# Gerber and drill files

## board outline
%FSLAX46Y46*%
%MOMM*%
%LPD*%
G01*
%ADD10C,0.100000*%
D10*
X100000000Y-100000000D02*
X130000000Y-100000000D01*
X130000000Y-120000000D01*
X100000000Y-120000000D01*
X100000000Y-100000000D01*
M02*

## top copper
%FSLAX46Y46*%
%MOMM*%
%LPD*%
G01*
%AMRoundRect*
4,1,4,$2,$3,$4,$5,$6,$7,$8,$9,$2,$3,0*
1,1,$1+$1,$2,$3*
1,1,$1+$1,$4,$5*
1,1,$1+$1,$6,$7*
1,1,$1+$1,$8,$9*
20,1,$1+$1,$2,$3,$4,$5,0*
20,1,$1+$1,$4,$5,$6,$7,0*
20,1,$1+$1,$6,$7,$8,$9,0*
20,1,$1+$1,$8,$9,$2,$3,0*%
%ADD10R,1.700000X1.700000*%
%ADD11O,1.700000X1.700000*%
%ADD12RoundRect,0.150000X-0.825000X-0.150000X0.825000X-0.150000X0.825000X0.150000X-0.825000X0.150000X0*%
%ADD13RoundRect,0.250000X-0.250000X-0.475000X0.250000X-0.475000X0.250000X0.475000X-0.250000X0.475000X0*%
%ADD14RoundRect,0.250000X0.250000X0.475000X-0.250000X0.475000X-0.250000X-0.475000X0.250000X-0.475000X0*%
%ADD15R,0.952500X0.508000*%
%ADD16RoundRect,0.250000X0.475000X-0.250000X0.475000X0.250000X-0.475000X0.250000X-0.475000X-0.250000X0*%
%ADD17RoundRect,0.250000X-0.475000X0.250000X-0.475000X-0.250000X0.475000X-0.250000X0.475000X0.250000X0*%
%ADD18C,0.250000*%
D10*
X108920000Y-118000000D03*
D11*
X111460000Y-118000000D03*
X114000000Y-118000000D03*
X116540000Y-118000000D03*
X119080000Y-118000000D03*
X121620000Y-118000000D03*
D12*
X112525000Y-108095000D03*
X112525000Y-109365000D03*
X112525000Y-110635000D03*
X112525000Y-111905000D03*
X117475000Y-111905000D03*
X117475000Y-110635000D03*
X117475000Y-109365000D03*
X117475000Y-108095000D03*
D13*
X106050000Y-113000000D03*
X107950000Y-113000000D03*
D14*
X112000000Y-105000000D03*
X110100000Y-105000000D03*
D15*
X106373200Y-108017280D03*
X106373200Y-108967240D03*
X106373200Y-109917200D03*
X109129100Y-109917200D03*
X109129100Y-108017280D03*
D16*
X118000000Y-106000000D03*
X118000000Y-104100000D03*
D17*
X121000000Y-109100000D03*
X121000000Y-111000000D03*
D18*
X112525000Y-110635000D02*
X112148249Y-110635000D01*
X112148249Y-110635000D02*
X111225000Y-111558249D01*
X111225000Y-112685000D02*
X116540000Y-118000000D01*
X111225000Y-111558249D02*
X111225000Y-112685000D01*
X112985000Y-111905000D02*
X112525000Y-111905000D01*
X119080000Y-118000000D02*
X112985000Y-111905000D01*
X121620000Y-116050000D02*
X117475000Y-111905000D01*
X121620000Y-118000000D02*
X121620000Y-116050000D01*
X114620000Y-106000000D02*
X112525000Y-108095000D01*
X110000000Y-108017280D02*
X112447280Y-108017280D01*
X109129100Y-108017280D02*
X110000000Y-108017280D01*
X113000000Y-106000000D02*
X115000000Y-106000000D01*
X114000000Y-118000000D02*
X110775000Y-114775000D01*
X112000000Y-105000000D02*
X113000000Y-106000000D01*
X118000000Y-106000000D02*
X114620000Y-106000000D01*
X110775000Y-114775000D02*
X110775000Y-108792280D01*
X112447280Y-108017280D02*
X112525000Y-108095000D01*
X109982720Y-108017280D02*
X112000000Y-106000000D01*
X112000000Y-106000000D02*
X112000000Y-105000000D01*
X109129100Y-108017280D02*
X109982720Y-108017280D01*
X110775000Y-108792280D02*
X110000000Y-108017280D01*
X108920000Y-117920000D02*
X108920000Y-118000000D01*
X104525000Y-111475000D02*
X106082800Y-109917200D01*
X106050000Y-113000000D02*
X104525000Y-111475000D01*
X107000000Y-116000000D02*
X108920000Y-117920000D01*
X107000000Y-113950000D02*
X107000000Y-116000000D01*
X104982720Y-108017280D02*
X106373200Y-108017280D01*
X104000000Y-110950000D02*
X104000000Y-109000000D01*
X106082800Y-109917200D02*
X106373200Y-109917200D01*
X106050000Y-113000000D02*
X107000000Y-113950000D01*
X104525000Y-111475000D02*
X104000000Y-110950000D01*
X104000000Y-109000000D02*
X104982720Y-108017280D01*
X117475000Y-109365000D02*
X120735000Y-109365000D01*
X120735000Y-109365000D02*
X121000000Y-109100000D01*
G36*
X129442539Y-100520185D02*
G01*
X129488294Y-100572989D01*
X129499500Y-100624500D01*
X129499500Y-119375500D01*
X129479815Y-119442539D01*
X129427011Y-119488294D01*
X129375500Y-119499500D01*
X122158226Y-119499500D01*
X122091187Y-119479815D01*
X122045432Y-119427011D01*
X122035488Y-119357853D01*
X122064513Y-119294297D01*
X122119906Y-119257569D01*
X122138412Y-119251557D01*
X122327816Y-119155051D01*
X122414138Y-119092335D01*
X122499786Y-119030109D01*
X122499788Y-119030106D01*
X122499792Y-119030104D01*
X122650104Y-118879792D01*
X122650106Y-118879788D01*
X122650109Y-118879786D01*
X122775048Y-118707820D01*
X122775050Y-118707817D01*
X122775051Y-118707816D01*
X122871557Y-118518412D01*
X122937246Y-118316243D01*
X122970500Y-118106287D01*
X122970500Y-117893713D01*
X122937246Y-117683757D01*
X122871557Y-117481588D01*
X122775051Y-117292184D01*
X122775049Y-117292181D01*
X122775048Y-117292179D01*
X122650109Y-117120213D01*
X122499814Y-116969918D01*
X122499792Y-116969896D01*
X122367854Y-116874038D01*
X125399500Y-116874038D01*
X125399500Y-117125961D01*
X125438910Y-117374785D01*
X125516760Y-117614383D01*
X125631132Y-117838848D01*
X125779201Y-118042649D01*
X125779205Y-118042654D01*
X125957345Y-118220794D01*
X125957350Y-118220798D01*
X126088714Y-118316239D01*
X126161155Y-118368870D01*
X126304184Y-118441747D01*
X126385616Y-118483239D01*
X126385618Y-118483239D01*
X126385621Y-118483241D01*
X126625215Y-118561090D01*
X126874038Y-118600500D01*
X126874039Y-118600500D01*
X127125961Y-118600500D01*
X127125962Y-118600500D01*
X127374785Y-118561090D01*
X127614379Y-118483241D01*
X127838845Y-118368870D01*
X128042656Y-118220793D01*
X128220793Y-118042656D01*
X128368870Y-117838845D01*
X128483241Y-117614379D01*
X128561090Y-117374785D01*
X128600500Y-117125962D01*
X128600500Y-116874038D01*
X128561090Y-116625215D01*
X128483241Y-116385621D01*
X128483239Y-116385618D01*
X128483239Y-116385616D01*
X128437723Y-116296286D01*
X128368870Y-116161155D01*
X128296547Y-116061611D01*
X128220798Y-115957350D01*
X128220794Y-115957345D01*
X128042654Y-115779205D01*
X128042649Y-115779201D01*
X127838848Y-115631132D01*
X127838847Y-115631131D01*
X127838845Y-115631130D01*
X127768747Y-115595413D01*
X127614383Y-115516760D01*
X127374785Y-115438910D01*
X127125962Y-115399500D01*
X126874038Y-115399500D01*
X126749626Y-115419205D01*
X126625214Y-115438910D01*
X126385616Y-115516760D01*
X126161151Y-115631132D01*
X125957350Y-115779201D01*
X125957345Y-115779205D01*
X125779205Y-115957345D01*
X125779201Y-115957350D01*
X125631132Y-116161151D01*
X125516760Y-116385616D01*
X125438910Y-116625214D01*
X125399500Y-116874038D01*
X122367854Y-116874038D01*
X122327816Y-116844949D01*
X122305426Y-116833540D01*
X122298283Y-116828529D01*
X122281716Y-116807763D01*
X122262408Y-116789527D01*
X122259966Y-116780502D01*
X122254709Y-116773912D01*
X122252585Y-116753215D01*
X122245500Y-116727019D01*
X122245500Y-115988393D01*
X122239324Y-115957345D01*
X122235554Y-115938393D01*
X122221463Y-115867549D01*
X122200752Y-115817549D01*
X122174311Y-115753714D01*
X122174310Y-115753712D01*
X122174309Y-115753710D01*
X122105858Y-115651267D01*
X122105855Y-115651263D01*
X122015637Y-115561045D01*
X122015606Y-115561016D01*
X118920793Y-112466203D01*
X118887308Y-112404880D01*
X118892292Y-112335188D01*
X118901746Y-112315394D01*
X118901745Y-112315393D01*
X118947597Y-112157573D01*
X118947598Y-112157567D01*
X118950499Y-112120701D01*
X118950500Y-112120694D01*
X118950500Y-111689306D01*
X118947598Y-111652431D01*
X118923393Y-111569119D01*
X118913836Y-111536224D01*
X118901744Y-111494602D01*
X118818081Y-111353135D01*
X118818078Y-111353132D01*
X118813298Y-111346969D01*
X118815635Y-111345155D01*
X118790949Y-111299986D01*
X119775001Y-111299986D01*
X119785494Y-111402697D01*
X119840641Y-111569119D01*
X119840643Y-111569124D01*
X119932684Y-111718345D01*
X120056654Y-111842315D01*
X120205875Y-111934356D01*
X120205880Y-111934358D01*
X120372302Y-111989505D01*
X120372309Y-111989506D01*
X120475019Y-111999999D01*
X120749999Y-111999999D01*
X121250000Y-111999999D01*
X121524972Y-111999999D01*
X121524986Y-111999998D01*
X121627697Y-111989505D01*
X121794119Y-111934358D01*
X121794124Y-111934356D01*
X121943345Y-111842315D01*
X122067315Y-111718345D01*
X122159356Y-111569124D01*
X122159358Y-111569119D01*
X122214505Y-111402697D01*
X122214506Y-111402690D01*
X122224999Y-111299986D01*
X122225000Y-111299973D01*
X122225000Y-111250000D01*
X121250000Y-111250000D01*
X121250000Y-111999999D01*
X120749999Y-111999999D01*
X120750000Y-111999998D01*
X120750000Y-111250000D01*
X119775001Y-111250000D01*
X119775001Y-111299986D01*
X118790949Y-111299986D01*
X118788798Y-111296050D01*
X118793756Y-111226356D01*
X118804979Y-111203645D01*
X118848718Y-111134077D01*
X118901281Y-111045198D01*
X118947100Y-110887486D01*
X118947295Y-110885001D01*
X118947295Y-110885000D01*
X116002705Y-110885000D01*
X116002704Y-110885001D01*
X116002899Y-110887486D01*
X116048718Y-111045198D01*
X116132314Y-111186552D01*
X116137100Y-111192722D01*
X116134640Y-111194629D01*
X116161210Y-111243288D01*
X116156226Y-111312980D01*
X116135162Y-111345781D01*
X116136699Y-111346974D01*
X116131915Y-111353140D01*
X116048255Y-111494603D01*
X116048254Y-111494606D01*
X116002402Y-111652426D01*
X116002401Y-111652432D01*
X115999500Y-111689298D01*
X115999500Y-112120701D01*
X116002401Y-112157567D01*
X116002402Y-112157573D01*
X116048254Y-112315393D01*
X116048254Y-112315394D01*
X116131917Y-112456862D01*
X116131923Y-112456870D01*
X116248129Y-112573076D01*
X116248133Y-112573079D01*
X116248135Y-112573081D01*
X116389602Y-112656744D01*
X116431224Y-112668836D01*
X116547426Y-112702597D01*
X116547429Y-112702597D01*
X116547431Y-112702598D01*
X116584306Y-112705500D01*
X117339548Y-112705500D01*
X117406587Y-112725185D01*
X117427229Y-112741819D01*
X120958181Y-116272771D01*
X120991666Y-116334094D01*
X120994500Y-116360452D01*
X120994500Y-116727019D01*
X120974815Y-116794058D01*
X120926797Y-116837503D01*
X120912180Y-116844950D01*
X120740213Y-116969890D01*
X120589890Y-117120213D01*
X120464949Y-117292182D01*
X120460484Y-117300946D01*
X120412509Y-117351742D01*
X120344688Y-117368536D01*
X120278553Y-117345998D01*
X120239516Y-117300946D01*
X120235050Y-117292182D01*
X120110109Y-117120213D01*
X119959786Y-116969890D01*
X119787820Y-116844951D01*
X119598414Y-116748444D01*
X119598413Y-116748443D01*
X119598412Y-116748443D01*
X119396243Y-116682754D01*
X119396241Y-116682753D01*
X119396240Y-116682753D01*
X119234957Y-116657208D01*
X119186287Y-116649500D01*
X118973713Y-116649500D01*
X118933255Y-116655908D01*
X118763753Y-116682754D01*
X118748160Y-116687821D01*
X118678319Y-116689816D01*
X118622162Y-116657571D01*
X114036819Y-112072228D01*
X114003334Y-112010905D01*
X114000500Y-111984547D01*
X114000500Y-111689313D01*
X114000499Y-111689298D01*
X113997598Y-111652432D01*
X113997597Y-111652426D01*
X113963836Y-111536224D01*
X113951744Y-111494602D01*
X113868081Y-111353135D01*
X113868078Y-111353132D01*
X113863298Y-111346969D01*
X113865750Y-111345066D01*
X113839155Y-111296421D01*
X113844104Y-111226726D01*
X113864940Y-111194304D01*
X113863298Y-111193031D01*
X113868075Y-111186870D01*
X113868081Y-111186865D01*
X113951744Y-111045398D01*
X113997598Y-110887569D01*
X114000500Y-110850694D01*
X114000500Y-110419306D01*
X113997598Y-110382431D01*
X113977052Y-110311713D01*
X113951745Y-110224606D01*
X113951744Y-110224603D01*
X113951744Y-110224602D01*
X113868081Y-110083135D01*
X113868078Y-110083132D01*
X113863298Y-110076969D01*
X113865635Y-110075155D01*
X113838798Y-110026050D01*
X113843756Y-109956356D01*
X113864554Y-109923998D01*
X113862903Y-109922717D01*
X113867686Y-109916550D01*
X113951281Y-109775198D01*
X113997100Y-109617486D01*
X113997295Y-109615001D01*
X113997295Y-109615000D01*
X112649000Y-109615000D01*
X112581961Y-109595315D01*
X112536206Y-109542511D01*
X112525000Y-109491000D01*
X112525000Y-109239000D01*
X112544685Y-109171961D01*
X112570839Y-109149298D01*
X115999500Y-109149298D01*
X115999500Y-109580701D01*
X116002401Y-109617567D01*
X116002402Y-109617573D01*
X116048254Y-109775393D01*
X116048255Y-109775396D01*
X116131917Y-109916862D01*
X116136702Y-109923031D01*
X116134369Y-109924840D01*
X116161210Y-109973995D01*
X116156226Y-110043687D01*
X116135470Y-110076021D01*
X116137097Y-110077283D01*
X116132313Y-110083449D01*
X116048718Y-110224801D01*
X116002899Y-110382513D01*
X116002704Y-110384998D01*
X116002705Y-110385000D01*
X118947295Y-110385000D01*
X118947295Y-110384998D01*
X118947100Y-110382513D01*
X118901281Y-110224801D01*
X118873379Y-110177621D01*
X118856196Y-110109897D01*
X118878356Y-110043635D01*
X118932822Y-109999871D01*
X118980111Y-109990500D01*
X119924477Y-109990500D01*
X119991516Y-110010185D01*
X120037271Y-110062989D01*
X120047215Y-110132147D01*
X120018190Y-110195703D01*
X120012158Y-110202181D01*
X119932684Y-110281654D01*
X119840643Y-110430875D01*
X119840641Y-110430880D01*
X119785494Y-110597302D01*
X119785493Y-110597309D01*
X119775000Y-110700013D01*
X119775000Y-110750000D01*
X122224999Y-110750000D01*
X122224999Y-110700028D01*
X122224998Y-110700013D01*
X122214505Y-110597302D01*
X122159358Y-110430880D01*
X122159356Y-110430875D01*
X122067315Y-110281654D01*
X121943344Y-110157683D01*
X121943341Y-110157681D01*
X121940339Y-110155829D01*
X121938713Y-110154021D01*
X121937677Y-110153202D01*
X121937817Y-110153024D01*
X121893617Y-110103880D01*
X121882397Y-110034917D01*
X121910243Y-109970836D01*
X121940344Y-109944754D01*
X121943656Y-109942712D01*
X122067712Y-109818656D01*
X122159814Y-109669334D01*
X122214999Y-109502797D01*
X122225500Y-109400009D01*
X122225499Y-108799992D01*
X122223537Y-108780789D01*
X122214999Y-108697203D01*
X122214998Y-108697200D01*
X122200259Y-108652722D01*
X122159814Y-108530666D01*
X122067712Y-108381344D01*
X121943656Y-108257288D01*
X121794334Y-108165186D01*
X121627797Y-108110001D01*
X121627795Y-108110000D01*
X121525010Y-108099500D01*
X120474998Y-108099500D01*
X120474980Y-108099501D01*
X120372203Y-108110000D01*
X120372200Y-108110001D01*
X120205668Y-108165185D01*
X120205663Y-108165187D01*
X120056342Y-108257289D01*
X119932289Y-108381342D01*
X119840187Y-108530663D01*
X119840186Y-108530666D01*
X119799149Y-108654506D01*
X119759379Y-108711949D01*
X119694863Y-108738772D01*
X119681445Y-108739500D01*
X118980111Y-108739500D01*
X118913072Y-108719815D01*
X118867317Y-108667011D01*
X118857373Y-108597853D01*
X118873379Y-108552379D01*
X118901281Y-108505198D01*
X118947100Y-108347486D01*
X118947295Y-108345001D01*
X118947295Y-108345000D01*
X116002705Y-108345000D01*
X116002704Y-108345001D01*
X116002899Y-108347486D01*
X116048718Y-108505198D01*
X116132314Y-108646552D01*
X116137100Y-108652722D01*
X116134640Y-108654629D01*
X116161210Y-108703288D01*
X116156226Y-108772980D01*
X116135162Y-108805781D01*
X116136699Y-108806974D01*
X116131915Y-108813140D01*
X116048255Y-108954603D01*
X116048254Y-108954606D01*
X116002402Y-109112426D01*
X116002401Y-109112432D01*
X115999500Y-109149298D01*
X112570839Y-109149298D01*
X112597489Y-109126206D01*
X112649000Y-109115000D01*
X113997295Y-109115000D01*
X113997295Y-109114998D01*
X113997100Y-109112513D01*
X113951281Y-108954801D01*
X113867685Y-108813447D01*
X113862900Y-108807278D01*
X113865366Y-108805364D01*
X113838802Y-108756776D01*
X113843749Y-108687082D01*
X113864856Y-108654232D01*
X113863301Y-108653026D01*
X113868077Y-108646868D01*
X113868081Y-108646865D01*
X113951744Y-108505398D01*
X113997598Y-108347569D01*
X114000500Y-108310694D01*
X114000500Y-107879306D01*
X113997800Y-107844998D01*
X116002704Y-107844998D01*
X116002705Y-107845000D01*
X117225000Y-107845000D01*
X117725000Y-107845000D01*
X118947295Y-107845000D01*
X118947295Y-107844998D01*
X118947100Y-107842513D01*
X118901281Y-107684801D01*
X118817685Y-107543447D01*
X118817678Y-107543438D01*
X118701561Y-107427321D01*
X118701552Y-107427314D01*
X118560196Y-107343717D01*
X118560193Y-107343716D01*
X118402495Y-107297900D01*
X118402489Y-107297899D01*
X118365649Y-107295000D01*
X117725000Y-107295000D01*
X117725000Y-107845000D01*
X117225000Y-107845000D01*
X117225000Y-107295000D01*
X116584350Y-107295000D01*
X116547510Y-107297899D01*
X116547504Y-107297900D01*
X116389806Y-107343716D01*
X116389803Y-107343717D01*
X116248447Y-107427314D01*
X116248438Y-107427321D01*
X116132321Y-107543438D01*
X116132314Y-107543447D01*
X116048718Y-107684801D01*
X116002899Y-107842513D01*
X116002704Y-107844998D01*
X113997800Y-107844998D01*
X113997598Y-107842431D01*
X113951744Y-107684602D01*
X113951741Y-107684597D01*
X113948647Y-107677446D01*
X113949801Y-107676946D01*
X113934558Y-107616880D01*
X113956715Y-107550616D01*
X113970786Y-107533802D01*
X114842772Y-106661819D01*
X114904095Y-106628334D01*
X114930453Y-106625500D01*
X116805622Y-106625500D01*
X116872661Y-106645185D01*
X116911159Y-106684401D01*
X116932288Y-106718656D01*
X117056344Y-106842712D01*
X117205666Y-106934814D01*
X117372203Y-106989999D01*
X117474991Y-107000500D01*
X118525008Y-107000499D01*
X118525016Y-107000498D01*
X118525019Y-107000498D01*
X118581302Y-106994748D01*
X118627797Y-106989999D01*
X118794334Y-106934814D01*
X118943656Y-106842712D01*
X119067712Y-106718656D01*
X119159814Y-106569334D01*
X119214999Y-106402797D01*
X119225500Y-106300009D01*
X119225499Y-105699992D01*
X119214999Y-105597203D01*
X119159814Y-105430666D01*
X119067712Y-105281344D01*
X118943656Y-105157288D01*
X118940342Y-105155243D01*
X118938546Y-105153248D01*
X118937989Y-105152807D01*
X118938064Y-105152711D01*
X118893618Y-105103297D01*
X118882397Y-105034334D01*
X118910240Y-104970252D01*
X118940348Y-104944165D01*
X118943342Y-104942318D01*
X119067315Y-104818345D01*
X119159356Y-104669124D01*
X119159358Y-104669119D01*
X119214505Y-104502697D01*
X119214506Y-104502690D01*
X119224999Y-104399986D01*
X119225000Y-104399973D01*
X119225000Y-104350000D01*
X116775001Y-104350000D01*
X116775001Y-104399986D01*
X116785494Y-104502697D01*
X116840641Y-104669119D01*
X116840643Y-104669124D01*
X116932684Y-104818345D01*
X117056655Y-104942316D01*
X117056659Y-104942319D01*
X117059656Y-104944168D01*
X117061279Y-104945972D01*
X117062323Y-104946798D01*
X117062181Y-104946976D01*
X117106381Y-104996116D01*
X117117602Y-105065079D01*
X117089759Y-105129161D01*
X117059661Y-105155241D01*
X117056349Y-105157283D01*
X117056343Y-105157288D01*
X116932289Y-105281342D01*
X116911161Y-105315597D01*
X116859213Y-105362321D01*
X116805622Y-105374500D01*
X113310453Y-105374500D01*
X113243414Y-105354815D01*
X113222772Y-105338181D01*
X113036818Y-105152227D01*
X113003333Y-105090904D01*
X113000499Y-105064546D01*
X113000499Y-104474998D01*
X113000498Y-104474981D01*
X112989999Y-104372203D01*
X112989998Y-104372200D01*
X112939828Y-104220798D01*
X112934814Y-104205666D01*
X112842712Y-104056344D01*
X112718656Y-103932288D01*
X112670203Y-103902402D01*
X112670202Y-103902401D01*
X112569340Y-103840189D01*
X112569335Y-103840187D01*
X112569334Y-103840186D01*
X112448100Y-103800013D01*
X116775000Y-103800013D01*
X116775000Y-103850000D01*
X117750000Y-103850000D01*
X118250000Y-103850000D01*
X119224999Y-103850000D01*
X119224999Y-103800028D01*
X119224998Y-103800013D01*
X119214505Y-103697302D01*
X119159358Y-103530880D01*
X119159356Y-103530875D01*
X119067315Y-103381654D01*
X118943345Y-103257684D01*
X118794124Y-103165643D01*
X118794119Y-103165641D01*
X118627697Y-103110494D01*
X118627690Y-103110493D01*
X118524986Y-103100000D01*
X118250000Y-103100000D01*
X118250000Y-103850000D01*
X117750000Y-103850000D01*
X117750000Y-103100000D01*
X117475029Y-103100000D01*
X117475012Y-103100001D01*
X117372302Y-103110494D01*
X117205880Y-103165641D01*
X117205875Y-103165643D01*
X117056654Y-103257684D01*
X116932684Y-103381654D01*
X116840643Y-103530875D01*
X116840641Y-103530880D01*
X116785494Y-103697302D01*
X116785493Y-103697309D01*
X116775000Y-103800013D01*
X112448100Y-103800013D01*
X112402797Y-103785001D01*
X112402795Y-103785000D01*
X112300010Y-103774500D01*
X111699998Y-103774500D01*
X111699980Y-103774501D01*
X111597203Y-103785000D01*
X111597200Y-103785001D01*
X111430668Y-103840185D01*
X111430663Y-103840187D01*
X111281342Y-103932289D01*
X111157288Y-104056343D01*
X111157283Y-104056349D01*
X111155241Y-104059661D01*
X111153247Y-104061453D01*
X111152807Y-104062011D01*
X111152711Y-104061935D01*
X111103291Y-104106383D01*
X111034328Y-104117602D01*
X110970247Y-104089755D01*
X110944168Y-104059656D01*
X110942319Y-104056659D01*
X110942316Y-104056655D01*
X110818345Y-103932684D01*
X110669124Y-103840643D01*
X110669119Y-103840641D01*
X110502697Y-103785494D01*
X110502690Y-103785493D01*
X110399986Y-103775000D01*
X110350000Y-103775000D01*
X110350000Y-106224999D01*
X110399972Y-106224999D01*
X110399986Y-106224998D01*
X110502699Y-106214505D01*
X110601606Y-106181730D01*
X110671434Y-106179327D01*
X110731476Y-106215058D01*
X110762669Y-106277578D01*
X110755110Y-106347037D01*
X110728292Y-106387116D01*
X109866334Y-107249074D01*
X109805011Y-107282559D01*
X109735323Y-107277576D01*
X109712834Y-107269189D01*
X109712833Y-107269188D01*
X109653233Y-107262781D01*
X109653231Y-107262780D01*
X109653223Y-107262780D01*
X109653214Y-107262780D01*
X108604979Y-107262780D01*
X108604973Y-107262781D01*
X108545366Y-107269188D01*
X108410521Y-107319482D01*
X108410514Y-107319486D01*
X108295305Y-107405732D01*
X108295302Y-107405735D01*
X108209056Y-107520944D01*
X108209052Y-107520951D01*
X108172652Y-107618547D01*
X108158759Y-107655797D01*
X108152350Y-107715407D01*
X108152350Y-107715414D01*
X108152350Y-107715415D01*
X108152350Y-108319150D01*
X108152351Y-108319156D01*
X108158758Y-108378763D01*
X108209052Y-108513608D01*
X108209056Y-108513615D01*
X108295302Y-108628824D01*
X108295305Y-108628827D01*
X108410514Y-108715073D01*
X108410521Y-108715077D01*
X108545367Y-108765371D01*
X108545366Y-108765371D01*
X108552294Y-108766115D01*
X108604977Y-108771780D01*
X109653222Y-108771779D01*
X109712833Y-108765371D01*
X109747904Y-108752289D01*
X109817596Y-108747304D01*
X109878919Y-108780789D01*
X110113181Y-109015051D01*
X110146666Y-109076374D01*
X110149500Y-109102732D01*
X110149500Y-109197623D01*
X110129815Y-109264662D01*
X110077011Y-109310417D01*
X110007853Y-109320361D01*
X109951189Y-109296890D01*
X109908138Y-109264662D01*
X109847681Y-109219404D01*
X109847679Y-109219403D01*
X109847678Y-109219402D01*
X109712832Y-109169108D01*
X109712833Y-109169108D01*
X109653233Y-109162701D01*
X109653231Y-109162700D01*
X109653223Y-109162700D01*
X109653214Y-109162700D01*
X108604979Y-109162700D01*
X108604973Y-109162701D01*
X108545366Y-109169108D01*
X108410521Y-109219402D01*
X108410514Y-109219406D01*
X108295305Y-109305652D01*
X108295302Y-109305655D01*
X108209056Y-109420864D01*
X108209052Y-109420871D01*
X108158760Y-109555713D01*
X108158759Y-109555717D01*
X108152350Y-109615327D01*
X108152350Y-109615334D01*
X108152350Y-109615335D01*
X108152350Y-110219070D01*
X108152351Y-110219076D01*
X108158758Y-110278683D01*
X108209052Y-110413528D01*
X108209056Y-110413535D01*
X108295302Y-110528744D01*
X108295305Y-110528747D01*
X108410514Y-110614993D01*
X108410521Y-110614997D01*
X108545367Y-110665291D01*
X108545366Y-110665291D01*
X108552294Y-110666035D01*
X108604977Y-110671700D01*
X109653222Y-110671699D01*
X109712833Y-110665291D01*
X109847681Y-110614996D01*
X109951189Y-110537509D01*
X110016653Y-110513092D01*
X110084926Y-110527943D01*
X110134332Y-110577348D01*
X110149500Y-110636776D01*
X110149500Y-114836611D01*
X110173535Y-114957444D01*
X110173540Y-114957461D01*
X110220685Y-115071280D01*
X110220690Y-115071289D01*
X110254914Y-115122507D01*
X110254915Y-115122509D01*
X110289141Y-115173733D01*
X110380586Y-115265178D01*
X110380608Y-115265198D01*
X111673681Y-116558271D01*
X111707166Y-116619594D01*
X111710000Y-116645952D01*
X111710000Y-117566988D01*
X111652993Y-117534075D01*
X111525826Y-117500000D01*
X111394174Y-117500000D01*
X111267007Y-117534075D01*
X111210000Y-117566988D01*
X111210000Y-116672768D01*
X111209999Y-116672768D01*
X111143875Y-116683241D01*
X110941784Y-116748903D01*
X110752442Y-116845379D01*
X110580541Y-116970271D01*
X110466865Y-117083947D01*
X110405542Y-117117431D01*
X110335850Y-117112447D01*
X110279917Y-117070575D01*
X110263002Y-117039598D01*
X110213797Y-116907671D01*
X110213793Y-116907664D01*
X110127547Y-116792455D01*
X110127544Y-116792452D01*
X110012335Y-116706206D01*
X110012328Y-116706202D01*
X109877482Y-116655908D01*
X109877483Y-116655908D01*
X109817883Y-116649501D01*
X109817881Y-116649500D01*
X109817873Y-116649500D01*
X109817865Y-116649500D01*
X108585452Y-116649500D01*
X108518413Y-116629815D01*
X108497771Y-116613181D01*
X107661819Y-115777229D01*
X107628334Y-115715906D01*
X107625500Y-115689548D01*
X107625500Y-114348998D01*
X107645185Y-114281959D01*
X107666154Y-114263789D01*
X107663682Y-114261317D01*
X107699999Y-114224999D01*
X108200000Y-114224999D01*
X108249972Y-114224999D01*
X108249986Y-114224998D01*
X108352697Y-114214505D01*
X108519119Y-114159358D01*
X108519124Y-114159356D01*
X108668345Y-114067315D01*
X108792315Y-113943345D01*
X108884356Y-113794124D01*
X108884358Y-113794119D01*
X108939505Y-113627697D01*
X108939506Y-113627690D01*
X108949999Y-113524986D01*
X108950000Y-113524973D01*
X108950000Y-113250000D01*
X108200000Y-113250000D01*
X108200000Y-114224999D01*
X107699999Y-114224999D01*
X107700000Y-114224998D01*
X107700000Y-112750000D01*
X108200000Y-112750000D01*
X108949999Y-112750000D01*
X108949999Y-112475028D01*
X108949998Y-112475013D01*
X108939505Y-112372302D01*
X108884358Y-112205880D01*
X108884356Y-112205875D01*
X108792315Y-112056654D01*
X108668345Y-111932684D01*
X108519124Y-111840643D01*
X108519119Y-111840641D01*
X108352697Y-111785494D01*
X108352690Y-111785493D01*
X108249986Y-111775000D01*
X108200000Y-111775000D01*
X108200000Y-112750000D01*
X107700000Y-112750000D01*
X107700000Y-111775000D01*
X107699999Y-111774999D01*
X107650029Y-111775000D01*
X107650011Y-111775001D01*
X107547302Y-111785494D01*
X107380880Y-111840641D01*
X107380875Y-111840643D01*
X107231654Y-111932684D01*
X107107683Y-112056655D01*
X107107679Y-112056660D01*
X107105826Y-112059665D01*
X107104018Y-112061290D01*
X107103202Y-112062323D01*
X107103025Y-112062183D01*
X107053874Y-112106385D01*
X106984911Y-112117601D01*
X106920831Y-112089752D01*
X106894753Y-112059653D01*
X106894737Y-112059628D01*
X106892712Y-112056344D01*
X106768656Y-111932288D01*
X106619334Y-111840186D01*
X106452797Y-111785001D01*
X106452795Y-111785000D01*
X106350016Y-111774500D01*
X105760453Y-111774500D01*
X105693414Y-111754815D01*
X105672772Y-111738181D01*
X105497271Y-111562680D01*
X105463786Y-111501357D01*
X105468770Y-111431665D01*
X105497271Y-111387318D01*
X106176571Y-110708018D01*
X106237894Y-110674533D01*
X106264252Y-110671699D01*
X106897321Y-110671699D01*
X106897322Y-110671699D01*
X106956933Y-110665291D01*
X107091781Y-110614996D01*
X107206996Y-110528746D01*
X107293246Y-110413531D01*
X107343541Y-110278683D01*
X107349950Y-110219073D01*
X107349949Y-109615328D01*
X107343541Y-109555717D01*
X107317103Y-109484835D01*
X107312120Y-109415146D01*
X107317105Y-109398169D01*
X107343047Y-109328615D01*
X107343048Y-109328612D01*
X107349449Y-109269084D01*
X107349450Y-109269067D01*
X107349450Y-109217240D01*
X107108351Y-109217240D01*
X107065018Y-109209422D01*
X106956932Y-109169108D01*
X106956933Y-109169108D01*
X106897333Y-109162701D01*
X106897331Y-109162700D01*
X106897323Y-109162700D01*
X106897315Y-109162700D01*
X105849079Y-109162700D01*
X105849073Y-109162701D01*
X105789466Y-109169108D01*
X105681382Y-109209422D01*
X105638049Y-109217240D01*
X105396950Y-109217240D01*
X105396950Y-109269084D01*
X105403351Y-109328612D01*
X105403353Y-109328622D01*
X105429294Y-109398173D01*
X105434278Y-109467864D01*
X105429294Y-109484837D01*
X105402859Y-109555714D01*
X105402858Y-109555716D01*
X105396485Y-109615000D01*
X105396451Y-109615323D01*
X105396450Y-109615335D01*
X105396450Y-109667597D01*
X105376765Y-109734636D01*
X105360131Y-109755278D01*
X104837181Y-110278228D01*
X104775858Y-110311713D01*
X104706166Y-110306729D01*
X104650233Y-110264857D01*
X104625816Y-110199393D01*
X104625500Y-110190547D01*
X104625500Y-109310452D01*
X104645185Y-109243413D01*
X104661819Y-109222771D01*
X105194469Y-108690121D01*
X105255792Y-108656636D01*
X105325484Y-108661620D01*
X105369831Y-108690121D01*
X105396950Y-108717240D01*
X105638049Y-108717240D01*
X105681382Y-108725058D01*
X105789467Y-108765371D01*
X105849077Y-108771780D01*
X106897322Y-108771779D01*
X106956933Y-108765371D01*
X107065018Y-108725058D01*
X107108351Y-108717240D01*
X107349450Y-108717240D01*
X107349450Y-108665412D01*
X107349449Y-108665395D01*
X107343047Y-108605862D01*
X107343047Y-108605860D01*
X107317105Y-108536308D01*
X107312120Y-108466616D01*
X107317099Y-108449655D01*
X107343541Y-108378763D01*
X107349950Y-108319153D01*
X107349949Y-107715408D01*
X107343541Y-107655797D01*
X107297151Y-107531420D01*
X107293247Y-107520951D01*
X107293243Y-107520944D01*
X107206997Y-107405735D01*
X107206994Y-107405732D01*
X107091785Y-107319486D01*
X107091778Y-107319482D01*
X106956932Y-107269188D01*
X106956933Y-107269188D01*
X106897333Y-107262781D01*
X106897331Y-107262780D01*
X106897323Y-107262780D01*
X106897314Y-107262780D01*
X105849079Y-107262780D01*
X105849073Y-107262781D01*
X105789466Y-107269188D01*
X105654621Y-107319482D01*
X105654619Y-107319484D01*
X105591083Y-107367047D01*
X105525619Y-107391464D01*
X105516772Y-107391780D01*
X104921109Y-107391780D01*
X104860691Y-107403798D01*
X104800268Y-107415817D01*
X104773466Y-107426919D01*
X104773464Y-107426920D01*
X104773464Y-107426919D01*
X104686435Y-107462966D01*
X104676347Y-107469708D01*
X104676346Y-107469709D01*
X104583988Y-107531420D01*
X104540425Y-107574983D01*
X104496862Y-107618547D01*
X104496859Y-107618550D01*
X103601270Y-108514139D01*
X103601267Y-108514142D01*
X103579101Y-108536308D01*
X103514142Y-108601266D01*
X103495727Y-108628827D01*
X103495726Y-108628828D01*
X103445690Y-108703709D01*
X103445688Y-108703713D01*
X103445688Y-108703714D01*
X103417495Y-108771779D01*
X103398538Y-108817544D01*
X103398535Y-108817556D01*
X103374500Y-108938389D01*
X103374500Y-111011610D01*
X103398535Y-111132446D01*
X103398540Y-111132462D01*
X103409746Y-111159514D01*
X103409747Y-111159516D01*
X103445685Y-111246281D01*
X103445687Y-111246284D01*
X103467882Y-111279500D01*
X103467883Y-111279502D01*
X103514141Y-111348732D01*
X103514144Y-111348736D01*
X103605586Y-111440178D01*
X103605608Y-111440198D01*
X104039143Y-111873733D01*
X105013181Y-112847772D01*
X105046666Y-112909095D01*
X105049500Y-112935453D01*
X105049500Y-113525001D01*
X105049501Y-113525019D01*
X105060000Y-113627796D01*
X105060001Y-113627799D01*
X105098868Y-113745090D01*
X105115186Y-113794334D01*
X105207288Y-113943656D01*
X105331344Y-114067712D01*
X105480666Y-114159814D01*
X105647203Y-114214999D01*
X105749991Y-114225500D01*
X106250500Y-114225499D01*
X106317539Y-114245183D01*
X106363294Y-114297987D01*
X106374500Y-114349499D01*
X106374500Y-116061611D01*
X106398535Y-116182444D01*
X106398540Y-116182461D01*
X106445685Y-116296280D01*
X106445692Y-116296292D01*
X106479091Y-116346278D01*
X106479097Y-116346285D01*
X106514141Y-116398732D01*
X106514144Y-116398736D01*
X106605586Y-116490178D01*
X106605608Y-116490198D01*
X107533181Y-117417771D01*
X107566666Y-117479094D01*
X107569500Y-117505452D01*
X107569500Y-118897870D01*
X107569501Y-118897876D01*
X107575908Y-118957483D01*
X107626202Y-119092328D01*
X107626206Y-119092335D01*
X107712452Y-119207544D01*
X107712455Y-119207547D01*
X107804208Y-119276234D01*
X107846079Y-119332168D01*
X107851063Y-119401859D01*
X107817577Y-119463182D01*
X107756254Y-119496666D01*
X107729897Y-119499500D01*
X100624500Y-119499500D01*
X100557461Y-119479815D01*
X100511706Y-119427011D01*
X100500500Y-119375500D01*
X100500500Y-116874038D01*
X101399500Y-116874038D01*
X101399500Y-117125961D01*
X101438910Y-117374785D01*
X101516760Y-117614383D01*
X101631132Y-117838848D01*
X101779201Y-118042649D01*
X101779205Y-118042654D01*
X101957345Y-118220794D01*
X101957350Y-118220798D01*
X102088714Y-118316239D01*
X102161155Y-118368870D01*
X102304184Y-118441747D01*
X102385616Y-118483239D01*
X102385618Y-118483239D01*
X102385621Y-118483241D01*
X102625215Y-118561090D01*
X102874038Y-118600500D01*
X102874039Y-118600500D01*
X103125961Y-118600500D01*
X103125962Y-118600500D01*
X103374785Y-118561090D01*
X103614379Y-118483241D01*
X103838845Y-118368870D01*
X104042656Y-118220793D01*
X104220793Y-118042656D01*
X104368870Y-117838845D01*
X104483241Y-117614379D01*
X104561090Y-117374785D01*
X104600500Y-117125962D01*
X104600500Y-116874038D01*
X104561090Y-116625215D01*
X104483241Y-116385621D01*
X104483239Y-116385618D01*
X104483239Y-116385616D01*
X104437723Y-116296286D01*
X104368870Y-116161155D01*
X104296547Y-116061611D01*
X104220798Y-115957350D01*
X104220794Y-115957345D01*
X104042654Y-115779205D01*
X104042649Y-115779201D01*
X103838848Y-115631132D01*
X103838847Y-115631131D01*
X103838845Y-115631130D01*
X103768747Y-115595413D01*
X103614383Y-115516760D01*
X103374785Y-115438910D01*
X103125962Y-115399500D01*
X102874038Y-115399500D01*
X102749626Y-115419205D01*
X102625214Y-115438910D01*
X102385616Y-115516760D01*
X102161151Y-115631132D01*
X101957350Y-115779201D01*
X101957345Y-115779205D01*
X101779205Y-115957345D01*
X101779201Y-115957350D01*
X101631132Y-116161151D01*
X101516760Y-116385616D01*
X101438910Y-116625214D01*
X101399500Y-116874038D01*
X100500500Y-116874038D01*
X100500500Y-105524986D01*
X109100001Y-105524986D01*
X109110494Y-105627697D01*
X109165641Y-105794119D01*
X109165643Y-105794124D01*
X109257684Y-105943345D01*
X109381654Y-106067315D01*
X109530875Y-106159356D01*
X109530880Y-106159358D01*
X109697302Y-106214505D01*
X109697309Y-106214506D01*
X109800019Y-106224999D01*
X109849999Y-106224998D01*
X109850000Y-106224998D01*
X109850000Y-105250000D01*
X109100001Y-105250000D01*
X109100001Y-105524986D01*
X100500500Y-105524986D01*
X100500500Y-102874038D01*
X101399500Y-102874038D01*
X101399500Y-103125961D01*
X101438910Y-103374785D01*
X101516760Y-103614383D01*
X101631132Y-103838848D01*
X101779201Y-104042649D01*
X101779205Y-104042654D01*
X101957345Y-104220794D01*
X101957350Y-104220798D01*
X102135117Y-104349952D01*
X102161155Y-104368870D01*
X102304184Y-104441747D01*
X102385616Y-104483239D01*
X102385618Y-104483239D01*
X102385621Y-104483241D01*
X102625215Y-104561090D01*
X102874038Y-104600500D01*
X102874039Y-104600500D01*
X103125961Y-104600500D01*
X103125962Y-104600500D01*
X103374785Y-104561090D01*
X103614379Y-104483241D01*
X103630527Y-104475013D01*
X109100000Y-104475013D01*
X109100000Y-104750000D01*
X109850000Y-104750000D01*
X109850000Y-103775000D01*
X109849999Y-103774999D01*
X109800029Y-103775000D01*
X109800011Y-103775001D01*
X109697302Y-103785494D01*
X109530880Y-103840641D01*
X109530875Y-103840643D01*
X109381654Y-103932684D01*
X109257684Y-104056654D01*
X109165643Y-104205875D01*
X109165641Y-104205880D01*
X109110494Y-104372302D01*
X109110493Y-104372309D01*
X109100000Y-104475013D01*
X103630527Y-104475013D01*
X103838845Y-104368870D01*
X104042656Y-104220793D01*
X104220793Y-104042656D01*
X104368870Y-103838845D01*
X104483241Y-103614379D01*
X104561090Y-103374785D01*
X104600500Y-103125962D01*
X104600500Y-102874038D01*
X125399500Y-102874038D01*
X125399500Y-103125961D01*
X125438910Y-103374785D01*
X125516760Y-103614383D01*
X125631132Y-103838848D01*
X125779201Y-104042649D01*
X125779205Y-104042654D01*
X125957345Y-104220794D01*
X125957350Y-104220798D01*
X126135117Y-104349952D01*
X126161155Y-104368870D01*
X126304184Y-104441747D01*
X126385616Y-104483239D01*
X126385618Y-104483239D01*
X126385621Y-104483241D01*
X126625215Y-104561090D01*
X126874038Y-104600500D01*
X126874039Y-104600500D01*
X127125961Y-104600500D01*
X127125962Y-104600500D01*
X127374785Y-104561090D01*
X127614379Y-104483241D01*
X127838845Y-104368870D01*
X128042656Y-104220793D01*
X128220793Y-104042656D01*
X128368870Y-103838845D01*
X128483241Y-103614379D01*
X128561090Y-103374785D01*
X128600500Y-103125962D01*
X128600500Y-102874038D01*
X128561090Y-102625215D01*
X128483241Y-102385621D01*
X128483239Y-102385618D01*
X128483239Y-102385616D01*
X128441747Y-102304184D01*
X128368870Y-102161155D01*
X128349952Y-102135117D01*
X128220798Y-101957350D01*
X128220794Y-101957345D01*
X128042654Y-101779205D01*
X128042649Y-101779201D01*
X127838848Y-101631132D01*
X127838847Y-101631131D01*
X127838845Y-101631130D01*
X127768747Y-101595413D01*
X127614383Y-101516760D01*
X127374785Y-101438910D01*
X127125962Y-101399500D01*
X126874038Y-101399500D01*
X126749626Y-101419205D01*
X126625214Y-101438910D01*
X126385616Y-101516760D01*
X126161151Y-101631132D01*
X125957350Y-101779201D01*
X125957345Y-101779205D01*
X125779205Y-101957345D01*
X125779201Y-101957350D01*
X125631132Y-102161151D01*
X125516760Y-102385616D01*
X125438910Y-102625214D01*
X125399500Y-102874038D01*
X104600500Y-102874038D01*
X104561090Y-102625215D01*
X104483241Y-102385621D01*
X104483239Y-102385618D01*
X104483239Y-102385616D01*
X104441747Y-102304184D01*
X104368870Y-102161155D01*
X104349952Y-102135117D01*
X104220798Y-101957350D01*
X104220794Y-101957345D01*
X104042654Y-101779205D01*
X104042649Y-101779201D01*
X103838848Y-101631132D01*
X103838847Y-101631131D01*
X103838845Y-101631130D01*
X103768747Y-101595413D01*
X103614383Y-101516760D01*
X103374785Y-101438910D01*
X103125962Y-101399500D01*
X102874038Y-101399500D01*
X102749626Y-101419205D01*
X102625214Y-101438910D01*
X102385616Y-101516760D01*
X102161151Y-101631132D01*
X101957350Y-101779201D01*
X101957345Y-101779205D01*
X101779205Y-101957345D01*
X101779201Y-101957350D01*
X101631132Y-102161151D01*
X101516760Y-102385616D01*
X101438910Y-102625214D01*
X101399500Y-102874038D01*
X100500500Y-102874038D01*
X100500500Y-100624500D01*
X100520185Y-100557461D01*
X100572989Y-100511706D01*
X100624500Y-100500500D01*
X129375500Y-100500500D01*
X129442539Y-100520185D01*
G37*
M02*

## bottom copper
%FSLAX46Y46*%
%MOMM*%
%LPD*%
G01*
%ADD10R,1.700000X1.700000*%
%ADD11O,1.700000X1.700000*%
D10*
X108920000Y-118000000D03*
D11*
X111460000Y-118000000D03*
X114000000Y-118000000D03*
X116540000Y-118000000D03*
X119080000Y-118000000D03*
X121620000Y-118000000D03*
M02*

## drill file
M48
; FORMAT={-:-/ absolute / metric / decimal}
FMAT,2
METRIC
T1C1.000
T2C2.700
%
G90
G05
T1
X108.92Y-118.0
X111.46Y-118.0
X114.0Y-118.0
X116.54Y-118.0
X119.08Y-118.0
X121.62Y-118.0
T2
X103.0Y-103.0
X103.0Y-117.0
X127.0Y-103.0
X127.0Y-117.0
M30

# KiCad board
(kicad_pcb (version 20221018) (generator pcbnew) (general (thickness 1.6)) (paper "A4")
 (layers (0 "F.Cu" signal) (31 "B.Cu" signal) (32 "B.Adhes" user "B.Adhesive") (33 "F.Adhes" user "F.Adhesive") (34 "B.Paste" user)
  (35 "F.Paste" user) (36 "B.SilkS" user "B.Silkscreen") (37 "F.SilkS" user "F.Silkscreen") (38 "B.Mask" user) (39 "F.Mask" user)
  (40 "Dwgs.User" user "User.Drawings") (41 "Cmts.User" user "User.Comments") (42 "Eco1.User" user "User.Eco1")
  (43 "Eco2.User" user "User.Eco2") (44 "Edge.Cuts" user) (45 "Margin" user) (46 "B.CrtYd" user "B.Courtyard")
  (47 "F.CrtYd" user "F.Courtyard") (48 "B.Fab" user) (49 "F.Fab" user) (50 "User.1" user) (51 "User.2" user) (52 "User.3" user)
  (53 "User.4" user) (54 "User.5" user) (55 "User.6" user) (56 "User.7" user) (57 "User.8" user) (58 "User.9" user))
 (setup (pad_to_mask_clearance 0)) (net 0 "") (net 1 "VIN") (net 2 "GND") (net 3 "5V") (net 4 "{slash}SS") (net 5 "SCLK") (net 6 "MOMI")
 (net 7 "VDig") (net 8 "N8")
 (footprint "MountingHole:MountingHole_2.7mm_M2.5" (layer "F.Cu") (at 103 117)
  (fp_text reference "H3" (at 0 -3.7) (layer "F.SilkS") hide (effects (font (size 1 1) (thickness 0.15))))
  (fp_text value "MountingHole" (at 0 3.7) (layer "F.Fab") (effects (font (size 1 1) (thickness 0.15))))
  (pad "" np_thru_hole circle (at 0 0) (size 2.7 2.7) (drill 2.7) (layers "*.Cu" "*.Mask")))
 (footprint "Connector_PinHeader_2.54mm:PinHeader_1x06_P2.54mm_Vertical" (layer "F.Cu") (at 108.92 118 90)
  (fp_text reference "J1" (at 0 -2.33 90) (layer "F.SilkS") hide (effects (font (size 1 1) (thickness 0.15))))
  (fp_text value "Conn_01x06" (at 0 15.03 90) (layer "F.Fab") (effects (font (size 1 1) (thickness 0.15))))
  (pad "1" thru_hole rect (at 0 0 90) (size 1.7 1.7) (drill 1) (layers "*.Cu" "*.Mask") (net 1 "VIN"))
  (pad "2" thru_hole oval (at 0 2.54 90) (size 1.7 1.7) (drill 1) (layers "*.Cu" "*.Mask") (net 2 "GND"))
  (pad "3" thru_hole oval (at 0 5.08 90) (size 1.7 1.7) (drill 1) (layers "*.Cu" "*.Mask") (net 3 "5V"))
  (pad "4" thru_hole oval (at 0 7.62 90) (size 1.7 1.7) (drill 1) (layers "*.Cu" "*.Mask") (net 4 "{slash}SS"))
  (pad "5" thru_hole oval (at 0 10.16 90) (size 1.7 1.7) (drill 1) (layers "*.Cu" "*.Mask") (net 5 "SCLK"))
  (pad "6" thru_hole oval (at 0 12.7 90) (size 1.7 1.7) (drill 1) (layers "*.Cu" "*.Mask") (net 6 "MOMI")))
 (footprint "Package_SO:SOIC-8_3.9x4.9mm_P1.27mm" (layer "F.Cu") (at 115 110)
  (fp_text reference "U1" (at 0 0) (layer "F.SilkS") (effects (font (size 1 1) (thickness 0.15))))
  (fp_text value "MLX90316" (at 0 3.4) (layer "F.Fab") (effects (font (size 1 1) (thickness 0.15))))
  (pad "1" smd roundrect (at -2.475 -1.905) (size 1.95 0.6) (layers "F.Cu" "F.Paste" "F.Mask") (roundrect_rratio 0.25) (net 3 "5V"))
  (pad "2" smd roundrect (at -2.475 -0.635) (size 1.95 0.6) (layers "F.Cu" "F.Paste" "F.Mask") (roundrect_rratio 0.25) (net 2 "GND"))
  (pad "3" smd roundrect (at -2.475 0.635) (size 1.95 0.6) (layers "F.Cu" "F.Paste" "F.Mask") (roundrect_rratio 0.25) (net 4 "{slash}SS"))
  (pad "4" smd roundrect (at -2.475 1.905) (size 1.95 0.6) (layers "F.Cu" "F.Paste" "F.Mask") (roundrect_rratio 0.25) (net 5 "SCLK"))
  (pad "5" smd roundrect (at 2.475 1.905) (size 1.95 0.6) (layers "F.Cu" "F.Paste" "F.Mask") (roundrect_rratio 0.25) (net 6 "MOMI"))
  (pad "6" smd roundrect (at 2.475 0.635) (size 1.95 0.6) (layers "F.Cu" "F.Paste" "F.Mask") (roundrect_rratio 0.25) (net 2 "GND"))
  (pad "7" smd roundrect (at 2.475 -0.635) (size 1.95 0.6) (layers "F.Cu" "F.Paste" "F.Mask") (roundrect_rratio 0.25) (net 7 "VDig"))
  (pad "8" smd roundrect (at 2.475 -1.905) (size 1.95 0.6) (layers "F.Cu" "F.Paste" "F.Mask") (roundrect_rratio 0.25) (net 2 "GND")))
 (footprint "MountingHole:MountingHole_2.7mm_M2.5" (layer "F.Cu") (at 127 103)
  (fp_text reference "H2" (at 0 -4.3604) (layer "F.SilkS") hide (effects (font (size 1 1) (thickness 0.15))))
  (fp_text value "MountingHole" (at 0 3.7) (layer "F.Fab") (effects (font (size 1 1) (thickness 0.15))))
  (pad "" np_thru_hole circle (at 0 0) (size 2.7 2.7) (drill 2.7) (layers "*.Cu" "*.Mask")))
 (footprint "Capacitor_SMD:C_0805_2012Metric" (layer "F.Cu") (at 107 113)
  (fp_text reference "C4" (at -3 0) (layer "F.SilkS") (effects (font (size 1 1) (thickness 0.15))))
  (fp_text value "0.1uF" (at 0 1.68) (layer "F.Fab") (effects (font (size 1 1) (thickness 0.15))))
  (pad "1" smd roundrect (at -0.95 0) (size 1 1.45) (layers "F.Cu" "F.Paste" "F.Mask") (roundrect_rratio 0.25) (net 1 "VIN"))
  (pad "2" smd roundrect (at 0.95 0) (size 1 1.45) (layers "F.Cu" "F.Paste" "F.Mask") (roundrect_rratio 0.25) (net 2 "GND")))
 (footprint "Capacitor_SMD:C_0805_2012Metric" (layer "F.Cu") (at 111.05 105 180)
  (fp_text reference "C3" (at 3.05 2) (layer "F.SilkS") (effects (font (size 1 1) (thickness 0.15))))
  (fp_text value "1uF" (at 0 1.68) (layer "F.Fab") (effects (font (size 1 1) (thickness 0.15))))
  (pad "1" smd roundrect (at -0.95 0 180) (size 1 1.45) (layers "F.Cu" "F.Paste" "F.Mask") (roundrect_rratio 0.25) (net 3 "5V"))
  (pad "2" smd roundrect (at 0.95 0 180) (size 1 1.45) (layers "F.Cu" "F.Paste" "F.Mask") (roundrect_rratio 0.25) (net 2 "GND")))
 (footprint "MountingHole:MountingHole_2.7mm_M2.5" (layer "F.Cu") (at 127 117)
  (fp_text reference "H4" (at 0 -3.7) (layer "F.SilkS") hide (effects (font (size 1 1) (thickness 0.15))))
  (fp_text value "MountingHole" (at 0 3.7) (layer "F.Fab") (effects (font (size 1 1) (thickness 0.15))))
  (pad "" np_thru_hole circle (at 0 0) (size 2.7 2.7) (drill 2.7) (layers "*.Cu" "*.Mask")))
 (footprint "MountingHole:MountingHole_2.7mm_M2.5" (layer "F.Cu") (at 103 103)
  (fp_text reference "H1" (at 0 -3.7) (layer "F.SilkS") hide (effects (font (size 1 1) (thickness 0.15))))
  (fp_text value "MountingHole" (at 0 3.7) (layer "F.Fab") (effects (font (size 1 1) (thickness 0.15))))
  (pad "" np_thru_hole circle (at 0 0) (size 2.7 2.7) (drill 2.7) (layers "*.Cu" "*.Mask")))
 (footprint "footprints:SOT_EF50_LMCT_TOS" (layer "F.Cu") (at 107.75115 108.96724)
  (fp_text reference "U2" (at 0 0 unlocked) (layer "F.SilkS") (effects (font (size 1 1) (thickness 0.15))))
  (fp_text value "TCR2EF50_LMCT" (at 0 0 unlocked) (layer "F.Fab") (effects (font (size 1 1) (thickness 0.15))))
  (pad "1" smd rect (at -1.37795 -0.94996) (size 0.9525 0.508) (layers "F.Cu" "F.Paste" "F.Mask") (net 1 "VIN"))
  (pad "2" smd rect (at -1.37795 0) (size 0.9525 0.508) (layers "F.Cu" "F.Paste" "F.Mask") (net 2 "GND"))
  (pad "3" smd rect (at -1.37795 0.94996) (size 0.9525 0.508) (layers "F.Cu" "F.Paste" "F.Mask") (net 1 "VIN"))
  (pad "4" smd rect (at 1.37795 0.94996) (size 0.9525 0.508) (layers "F.Cu" "F.Paste" "F.Mask") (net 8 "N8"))
  (pad "5" smd rect (at 1.37795 -0.94996) (size 0.9525 0.508) (layers "F.Cu" "F.Paste" "F.Mask") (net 3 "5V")))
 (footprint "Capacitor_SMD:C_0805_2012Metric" (layer "F.Cu") (at 118 105.05 90)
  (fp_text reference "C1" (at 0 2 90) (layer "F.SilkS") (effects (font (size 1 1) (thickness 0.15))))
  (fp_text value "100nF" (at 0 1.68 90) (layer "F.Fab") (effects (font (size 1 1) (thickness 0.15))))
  (pad "1" smd roundrect (at -0.95 0 90) (size 1 1.45) (layers "F.Cu" "F.Paste" "F.Mask") (roundrect_rratio 0.25) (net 3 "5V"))
  (pad "2" smd roundrect (at 0.95 0 90) (size 1 1.45) (layers "F.Cu" "F.Paste" "F.Mask") (roundrect_rratio 0.25) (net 2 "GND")))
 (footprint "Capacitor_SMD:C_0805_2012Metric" (layer "F.Cu") (at 121 110.05 -90)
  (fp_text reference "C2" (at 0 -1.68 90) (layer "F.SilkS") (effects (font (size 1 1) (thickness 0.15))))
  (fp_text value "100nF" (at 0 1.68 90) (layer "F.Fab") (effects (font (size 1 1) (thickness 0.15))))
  (pad "1" smd roundrect (at -0.95 0 270) (size 1 1.45) (layers "F.Cu" "F.Paste" "F.Mask") (roundrect_rratio 0.25) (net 7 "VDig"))
  (pad "2" smd roundrect (at 0.95 0 270) (size 1 1.45) (layers "F.Cu" "F.Paste" "F.Mask") (roundrect_rratio 0.25) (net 2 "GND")))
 (gr_rect (start 100 100) (end 130 120) (stroke (width 0.1) (type default)) (fill none) (layer "Edge.Cuts"))
 (segment (start 112.525 110.635) (end 112.148249 110.635) (width 0.25) (layer "F.Cu") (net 4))
 (segment (start 112.148249 110.635) (end 111.225 111.558249) (width 0.25) (layer "F.Cu") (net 4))
 (segment (start 111.225 112.685) (end 116.54 118) (width 0.25) (layer "F.Cu") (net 4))
 (segment (start 111.225 111.558249) (end 111.225 112.685) (width 0.25) (layer "F.Cu") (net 4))
 (segment (start 112.985 111.905) (end 112.525 111.905) (width 0.25) (layer "F.Cu") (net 5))
 (segment (start 119.08 118) (end 112.985 111.905) (width 0.25) (layer "F.Cu") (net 5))
 (segment (start 121.62 116.05) (end 117.475 111.905) (width 0.25) (layer "F.Cu") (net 6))
 (segment (start 121.62 118) (end 121.62 116.05) (width 0.25) (layer "F.Cu") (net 6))
 (segment (start 114.62 106) (end 112.525 108.095) (width 0.25) (layer "F.Cu") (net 3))
 (segment (start 110 108.01728) (end 112.44728 108.01728) (width 0.25) (layer "F.Cu") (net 3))
 (segment (start 109.1291 108.01728) (end 110 108.01728) (width 0.25) (layer "F.Cu") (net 3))
 (segment (start 113 106) (end 115 106) (width 0.25) (layer "F.Cu") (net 3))
 (segment (start 114 118) (end 110.775 114.775) (width 0.25) (layer "F.Cu") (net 3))
 (segment (start 112 105) (end 113 106) (width 0.25) (layer "F.Cu") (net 3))
 (segment (start 118 106) (end 114.62 106) (width 0.25) (layer "F.Cu") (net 3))
 (segment (start 110.775 114.775) (end 110.775 108.79228) (width 0.25) (layer "F.Cu") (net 3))
 (segment (start 112.44728 108.01728) (end 112.525 108.095) (width 0.25) (layer "F.Cu") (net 3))
 (segment (start 109.98272 108.01728) (end 112 106) (width 0.25) (layer "F.Cu") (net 3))
 (segment (start 112 106) (end 112 105) (width 0.25) (layer "F.Cu") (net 3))
 (segment (start 109.1291 108.01728) (end 109.98272 108.01728) (width 0.25) (layer "F.Cu") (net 3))
 (segment (start 110.775 108.79228) (end 110 108.01728) (width 0.25) (layer "F.Cu") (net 3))
 (segment (start 108.92 117.92) (end 108.92 118) (width 0.25) (layer "F.Cu") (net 1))
 (segment (start 104.525 111.475) (end 106.0828 109.9172) (width 0.25) (layer "F.Cu") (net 1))
 (segment (start 106.05 113) (end 104.525 111.475) (width 0.25) (layer "F.Cu") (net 1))
 (segment (start 107 116) (end 108.92 117.92) (width 0.25) (layer "F.Cu") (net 1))
 (segment (start 107 113.95) (end 107 116) (width 0.25) (layer "F.Cu") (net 1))
 (segment (start 104.98272 108.01728) (end 106.3732 108.01728) (width 0.25) (layer "F.Cu") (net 1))
 (segment (start 104 110.95) (end 104 109) (width 0.25) (layer "F.Cu") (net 1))
 (segment (start 106.0828 109.9172) (end 106.3732 109.9172) (width 0.25) (layer "F.Cu") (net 1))
 (segment (start 106.05 113) (end 107 113.95) (width 0.25) (layer "F.Cu") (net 1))
 (segment (start 104.525 111.475) (end 104 110.95) (width 0.25) (layer "F.Cu") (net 1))
 (segment (start 104 109) (end 104.98272 108.01728) (width 0.25) (layer "F.Cu") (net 1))
 (segment (start 117.475 109.365) (end 120.735 109.365) (width 0.25) (layer "F.Cu") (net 7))
 (segment (start 120.735 109.365) (end 121 109.1) (width 0.25) (layer "F.Cu") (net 7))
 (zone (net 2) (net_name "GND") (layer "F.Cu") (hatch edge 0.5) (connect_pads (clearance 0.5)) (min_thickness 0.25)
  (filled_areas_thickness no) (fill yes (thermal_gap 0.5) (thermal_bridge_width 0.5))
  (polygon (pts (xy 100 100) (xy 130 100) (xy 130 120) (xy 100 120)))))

